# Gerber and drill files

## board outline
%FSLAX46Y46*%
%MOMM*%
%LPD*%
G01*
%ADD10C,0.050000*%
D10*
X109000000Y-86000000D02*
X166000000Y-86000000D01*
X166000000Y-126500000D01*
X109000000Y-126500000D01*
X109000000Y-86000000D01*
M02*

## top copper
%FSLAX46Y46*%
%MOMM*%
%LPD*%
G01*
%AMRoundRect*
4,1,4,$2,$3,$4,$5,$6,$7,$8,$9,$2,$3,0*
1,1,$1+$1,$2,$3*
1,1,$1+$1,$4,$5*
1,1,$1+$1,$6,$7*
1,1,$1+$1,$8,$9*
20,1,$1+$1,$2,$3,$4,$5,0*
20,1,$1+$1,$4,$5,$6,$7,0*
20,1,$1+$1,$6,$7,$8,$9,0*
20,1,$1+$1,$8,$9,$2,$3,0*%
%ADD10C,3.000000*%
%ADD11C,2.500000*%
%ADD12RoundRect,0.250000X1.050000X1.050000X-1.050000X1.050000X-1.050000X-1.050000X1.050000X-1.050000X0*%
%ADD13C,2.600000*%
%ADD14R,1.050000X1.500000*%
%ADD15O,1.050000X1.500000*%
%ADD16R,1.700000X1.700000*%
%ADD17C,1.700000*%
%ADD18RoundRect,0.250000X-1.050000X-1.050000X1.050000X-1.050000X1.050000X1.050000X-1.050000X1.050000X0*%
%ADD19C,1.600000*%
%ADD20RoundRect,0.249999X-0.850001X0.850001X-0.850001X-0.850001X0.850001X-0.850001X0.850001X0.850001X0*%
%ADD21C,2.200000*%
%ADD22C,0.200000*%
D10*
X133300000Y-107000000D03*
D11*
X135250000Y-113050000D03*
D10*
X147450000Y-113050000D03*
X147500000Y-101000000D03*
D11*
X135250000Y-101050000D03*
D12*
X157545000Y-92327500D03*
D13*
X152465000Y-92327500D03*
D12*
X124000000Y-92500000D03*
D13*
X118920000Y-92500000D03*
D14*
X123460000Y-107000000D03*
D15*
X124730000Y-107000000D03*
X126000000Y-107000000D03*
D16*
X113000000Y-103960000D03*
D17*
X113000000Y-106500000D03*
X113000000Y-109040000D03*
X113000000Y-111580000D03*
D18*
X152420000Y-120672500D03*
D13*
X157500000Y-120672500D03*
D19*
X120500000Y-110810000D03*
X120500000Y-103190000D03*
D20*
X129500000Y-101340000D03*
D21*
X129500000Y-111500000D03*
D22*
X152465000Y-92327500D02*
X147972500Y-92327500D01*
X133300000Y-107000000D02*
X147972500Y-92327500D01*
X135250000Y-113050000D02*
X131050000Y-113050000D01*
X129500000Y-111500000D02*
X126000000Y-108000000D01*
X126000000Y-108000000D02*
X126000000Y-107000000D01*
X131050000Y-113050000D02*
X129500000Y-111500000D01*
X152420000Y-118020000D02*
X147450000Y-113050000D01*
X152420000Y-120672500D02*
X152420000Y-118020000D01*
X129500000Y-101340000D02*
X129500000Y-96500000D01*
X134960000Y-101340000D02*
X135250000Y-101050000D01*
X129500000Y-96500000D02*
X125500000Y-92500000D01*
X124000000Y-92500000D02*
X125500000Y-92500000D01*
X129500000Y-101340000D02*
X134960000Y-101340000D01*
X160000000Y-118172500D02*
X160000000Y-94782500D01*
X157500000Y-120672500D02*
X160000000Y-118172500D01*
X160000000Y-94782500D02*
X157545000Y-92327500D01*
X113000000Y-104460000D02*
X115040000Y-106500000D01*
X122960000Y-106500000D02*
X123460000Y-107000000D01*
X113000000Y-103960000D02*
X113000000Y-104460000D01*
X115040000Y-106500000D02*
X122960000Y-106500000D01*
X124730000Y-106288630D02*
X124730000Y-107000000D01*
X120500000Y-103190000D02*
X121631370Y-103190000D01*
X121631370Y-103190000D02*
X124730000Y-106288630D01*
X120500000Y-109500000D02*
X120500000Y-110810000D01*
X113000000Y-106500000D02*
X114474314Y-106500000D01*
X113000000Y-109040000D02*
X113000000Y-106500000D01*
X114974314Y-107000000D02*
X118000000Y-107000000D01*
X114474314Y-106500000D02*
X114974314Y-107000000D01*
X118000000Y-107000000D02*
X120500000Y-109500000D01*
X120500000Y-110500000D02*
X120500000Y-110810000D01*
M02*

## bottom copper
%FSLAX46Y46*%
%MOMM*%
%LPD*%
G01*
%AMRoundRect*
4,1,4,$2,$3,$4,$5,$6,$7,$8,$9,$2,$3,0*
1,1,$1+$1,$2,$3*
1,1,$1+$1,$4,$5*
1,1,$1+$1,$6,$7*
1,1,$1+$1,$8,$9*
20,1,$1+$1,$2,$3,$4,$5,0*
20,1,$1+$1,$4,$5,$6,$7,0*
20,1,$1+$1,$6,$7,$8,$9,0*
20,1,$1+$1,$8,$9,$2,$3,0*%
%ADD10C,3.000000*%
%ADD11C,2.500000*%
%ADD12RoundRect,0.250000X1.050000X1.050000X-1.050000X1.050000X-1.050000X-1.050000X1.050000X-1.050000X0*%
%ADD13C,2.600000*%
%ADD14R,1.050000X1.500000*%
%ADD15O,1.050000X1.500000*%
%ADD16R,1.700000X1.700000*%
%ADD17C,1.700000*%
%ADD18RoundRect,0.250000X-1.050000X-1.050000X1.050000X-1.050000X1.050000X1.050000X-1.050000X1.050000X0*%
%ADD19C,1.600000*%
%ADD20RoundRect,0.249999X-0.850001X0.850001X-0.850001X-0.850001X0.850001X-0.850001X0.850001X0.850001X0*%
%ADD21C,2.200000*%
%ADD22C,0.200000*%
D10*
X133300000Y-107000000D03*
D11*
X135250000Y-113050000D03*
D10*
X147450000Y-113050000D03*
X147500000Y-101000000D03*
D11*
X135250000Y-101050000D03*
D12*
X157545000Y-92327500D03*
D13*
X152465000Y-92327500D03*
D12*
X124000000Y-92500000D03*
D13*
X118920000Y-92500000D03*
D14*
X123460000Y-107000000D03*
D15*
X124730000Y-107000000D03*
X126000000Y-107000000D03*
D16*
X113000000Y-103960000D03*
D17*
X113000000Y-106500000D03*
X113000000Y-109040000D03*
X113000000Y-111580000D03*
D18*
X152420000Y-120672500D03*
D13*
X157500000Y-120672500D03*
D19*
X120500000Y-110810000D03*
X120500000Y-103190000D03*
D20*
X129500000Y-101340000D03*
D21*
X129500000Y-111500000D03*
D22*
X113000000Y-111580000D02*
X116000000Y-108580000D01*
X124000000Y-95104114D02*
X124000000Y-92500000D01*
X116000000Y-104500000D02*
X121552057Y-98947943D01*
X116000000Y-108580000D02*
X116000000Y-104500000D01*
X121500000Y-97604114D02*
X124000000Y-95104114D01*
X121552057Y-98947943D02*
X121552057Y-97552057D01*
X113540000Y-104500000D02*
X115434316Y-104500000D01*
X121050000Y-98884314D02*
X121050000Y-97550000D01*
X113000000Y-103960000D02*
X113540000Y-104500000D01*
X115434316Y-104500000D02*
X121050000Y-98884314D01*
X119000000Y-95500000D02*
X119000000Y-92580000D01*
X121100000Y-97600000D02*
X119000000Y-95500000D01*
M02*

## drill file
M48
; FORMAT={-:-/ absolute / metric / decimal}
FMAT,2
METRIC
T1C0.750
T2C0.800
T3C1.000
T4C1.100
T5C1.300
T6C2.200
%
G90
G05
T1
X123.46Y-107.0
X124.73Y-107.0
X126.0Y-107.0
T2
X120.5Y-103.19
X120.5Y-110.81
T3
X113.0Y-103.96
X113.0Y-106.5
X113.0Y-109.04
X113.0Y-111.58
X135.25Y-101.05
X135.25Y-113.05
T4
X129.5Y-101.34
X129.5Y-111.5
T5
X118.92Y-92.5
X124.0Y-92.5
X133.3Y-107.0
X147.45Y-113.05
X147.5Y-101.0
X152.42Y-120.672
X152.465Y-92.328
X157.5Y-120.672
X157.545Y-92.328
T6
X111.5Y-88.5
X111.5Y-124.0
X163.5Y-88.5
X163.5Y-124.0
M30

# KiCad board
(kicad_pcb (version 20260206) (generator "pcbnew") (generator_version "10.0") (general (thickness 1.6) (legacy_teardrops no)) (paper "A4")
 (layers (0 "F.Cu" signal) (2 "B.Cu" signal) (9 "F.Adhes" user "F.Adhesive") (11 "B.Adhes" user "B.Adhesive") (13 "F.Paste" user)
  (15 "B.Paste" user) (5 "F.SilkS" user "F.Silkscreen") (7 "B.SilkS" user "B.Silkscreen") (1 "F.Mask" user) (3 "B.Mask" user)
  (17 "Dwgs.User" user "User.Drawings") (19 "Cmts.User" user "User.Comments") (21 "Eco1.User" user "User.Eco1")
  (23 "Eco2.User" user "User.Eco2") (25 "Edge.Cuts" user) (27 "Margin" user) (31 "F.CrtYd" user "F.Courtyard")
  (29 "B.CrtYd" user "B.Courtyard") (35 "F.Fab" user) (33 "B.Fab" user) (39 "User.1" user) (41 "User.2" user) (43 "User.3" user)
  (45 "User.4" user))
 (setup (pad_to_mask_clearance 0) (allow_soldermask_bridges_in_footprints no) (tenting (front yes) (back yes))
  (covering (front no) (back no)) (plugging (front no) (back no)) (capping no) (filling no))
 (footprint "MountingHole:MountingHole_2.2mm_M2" (layer "F.Cu") (at 163.5 124)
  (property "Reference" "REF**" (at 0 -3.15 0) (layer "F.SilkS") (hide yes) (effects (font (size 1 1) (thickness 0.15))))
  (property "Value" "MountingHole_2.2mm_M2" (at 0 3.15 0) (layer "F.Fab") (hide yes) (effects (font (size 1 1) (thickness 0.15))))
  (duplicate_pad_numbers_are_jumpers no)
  (pad "" np_thru_hole circle (at 0 0) (size 2.2 2.2) (drill 2.2) (layers "*.Cu" "*.Mask")))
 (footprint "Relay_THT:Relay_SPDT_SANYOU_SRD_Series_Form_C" (layer "F.Cu") (at 133.3 107)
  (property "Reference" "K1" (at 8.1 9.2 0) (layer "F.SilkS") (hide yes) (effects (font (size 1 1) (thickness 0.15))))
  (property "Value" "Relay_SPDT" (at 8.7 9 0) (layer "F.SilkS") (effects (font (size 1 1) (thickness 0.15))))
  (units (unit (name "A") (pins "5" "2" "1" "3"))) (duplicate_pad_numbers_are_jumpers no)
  (pad "1" thru_hole circle (at 0 0 90) (size 3 3) (drill 1.3) (layers "*.Cu" "*.Mask") (remove_unused_layers no) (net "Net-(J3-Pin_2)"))
  (pad "2" thru_hole circle (at 1.95 6.05 90) (size 2.5 2.5) (drill 1) (layers "*.Cu" "*.Mask") (remove_unused_layers no) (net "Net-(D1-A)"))
  (pad "3" thru_hole circle (at 14.15 6.05 90) (size 3 3) (drill 1.3) (layers "*.Cu" "*.Mask") (remove_unused_layers no)
   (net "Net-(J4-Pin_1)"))
  (pad "4" thru_hole circle (at 14.2 -6 90) (size 3 3) (drill 1.3) (layers "*.Cu" "*.Mask") (remove_unused_layers no))
  (pad "5" thru_hole circle (at 1.95 -5.95 90) (size 2.5 2.5) (drill 1) (layers "*.Cu" "*.Mask") (remove_unused_layers no) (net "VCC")))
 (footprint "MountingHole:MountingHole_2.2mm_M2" (layer "F.Cu") (at 111.5 124)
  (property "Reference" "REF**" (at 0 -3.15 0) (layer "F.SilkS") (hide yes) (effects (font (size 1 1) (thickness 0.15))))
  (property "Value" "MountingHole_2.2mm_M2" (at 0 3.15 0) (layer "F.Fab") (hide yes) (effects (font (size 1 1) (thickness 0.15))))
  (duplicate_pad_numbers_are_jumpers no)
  (pad "" np_thru_hole circle (at 0 0) (size 2.2 2.2) (drill 2.2) (layers "*.Cu" "*.Mask")))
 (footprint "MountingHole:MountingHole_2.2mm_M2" (layer "F.Cu") (at 163.5 88.5)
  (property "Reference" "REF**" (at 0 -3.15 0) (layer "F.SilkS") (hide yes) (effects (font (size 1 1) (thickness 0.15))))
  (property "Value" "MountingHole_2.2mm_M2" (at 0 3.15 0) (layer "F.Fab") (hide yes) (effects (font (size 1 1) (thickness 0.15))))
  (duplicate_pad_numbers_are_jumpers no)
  (pad "" np_thru_hole circle (at 0 0) (size 2.2 2.2) (drill 2.2) (layers "*.Cu" "*.Mask")))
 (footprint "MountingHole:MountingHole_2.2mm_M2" (layer "F.Cu") (at 111.5 88.5)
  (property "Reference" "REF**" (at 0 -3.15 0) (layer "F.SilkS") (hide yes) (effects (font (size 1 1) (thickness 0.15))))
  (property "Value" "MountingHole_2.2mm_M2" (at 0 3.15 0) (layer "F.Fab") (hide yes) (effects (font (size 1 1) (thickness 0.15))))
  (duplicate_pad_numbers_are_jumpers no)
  (pad "" np_thru_hole circle (at 0 0) (size 2.2 2.2) (drill 2.2) (layers "*.Cu" "*.Mask")))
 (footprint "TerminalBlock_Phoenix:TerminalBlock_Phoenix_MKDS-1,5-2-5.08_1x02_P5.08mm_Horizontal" (layer "F.Cu") (at 157.545 92.3275 180)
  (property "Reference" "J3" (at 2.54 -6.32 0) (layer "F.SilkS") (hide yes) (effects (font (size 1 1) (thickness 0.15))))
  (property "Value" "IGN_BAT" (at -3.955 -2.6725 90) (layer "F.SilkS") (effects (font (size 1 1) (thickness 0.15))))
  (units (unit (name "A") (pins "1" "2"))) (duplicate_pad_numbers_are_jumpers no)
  (pad "1" thru_hole roundrect (at 0 0 180) (size 2.6 2.6) (drill 1.3) (layers "*.Cu" "*.Mask") (remove_unused_layers no)
   (roundrect_rratio 0.096154) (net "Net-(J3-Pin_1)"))
  (pad "2" thru_hole circle (at 5.08 0 180) (size 2.6 2.6) (drill 1.3) (layers "*.Cu" "*.Mask") (remove_unused_layers no)
   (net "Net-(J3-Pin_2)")))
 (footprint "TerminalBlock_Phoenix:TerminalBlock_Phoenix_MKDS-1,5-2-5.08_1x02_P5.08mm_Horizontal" (layer "F.Cu") (at 124 92.5 180)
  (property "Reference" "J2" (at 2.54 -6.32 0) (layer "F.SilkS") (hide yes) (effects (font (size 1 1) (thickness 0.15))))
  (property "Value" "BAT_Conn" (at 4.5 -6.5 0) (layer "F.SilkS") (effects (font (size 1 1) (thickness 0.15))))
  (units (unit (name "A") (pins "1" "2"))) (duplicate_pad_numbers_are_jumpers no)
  (pad "1" thru_hole roundrect (at 0 0 180) (size 2.6 2.6) (drill 1.3) (layers "*.Cu" "*.Mask") (remove_unused_layers no)
   (roundrect_rratio 0.096154) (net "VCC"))
  (pad "2" thru_hole circle (at 5.08 0 180) (size 2.6 2.6) (drill 1.3) (layers "*.Cu" "*.Mask") (remove_unused_layers no) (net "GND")))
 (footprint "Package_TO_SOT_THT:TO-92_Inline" (layer "F.Cu") (at 123.46 107)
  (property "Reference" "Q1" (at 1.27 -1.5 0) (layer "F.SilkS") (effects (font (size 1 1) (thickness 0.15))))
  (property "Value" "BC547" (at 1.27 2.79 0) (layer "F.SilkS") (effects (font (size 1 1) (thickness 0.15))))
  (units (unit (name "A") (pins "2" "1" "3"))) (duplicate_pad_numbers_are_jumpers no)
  (pad "1" thru_hole rect (at 0 0) (size 1.05 1.5) (drill 0.75) (layers "*.Cu" "*.Mask") (remove_unused_layers no) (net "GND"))
  (pad "2" thru_hole oval (at 1.27 0) (size 1.05 1.5) (drill 0.75) (layers "*.Cu" "*.Mask") (remove_unused_layers no) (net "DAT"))
  (pad "3" thru_hole oval (at 2.54 0) (size 1.05 1.5) (drill 0.75) (layers "*.Cu" "*.Mask") (remove_unused_layers no) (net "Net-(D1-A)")))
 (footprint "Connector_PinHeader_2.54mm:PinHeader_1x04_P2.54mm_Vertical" (layer "F.Cu") (at 113 103.96)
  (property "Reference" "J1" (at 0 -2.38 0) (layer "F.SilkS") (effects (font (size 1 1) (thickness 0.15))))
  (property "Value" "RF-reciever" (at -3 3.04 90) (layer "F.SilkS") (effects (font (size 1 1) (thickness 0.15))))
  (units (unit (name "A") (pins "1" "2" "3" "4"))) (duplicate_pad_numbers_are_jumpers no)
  (pad "1" thru_hole rect (at 0 0) (size 1.7 1.7) (drill 1) (layers "*.Cu" "*.Mask") (remove_unused_layers no) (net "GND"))
  (pad "2" thru_hole circle (at 0 2.54) (size 1.7 1.7) (drill 1) (layers "*.Cu" "*.Mask") (remove_unused_layers no) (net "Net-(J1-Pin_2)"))
  (pad "3" thru_hole circle (at 0 5.08) (size 1.7 1.7) (drill 1) (layers "*.Cu" "*.Mask") (remove_unused_layers no) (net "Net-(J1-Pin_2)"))
  (pad "4" thru_hole circle (at 0 7.62) (size 1.7 1.7) (drill 1) (layers "*.Cu" "*.Mask") (remove_unused_layers no) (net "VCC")))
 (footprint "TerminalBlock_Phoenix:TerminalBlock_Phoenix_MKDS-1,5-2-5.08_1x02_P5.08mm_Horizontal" (layer "F.Cu") (at 152.42 120.6725)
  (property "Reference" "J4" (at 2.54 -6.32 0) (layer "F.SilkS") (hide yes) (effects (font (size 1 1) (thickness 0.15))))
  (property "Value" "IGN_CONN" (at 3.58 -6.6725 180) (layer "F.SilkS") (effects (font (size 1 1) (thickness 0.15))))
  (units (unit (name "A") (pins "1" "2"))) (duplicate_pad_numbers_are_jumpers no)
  (pad "1" thru_hole roundrect (at 0 0) (size 2.6 2.6) (drill 1.3) (layers "*.Cu" "*.Mask") (remove_unused_layers no)
   (roundrect_rratio 0.096154) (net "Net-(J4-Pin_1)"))
  (pad "2" thru_hole circle (at 5.08 0) (size 2.6 2.6) (drill 1.3) (layers "*.Cu" "*.Mask") (remove_unused_layers no) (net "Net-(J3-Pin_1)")))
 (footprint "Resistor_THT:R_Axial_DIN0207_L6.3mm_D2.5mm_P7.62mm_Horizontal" (layer "F.Cu") (at 120.5 110.81 90)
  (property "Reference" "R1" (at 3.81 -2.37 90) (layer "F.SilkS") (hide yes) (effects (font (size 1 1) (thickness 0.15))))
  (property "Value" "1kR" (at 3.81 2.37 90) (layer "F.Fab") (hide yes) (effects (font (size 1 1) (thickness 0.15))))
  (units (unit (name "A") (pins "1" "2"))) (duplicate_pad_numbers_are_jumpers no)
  (pad "1" thru_hole circle (at 0 0 90) (size 1.6 1.6) (drill 0.8) (layers "*.Cu" "*.Mask") (remove_unused_layers no) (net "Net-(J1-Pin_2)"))
  (pad "2" thru_hole circle (at 7.62 0 90) (size 1.6 1.6) (drill 0.8) (layers "*.Cu" "*.Mask") (remove_unused_layers no) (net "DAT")))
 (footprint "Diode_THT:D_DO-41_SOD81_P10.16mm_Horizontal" (layer "F.Cu") (at 129.5 101.34 -90)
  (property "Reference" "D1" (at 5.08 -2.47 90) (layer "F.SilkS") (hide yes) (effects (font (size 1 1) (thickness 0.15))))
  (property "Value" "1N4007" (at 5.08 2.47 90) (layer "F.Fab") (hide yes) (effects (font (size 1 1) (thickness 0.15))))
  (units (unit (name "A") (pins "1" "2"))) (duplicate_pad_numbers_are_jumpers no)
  (pad "1" thru_hole roundrect (at 0 0 270) (size 2.2 2.2) (drill 1.1) (layers "*.Cu" "*.Mask") (remove_unused_layers no)
   (roundrect_rratio 0.113636) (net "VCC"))
  (pad "2" thru_hole circle (at 10.16 0 270) (size 2.2 2.2) (drill 1.1) (layers "*.Cu" "*.Mask") (remove_unused_layers no)
   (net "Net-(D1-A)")))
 (gr_rect (start 109 86) (end 166 126.5) (stroke (width 0.05) (type default)) (fill no) (layer "Edge.Cuts"))
 (segment (start 152.465 92.3275) (end 147.9725 92.3275) (width 0.2) (layer "F.Cu") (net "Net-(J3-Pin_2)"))
 (segment (start 133.3 107) (end 147.9725 92.3275) (width 0.2) (layer "F.Cu") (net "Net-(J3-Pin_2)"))
 (segment (start 135.25 113.05) (end 131.05 113.05) (width 0.2) (layer "F.Cu") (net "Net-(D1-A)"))
 (segment (start 129.5 111.5) (end 126 108) (width 0.2) (layer "F.Cu") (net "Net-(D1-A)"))
 (segment (start 126 108) (end 126 107) (width 0.2) (layer "F.Cu") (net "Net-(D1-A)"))
 (segment (start 131.05 113.05) (end 129.5 111.5) (width 0.2) (layer "F.Cu") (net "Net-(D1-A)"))
 (segment (start 152.42 118.02) (end 147.45 113.05) (width 0.2) (layer "F.Cu") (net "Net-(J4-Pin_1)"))
 (segment (start 152.42 120.6725) (end 152.42 118.02) (width 0.2) (layer "F.Cu") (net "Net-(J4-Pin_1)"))
 (segment (start 129.5 101.34) (end 129.5 96.5) (width 0.2) (layer "F.Cu") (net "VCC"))
 (segment (start 134.96 101.34) (end 135.25 101.05) (width 0.2) (layer "F.Cu") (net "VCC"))
 (segment (start 129.5 96.5) (end 125.5 92.5) (width 0.2) (layer "F.Cu") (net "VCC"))
 (segment (start 124 92.5) (end 125.5 92.5) (width 0.2) (layer "F.Cu") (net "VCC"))
 (segment (start 129.5 101.34) (end 134.96 101.34) (width 0.2) (layer "F.Cu") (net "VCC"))
 (segment (start 113 111.58) (end 116 108.58) (width 0.2) (layer "B.Cu") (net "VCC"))
 (segment (start 124 95.104114) (end 124 92.5) (width 0.2) (layer "B.Cu") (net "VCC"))
 (segment (start 116 104.5) (end 121.552057 98.947943) (width 0.2) (layer "B.Cu") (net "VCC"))
 (segment (start 116 108.58) (end 116 104.5) (width 0.2) (layer "B.Cu") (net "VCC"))
 (segment (start 121.5 97.604114) (end 124 95.104114) (width 0.2) (layer "B.Cu") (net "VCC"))
 (segment (start 121.552057 98.947943) (end 121.552057 97.552057) (width 0.2) (layer "B.Cu") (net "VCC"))
 (segment (start 160 118.1725) (end 160 94.7825) (width 0.2) (layer "F.Cu") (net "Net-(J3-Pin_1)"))
 (segment (start 157.5 120.6725) (end 160 118.1725) (width 0.2) (layer "F.Cu") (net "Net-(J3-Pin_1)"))
 (segment (start 160 94.7825) (end 157.545 92.3275) (width 0.2) (layer "F.Cu") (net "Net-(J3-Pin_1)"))
 (segment (start 113 104.46) (end 115.04 106.5) (width 0.2) (layer "F.Cu") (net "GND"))
 (segment (start 122.96 106.5) (end 123.46 107) (width 0.2) (layer "F.Cu") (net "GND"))
 (segment (start 113 103.96) (end 113 104.46) (width 0.2) (layer "F.Cu") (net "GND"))
 (segment (start 115.04 106.5) (end 122.96 106.5) (width 0.2) (layer "F.Cu") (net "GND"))
 (segment (start 113.54 104.5) (end 115.434316 104.5) (width 0.2) (layer "B.Cu") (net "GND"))
 (segment (start 121.05 98.884314) (end 121.05 97.55) (width 0.2) (layer "B.Cu") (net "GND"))
 (segment (start 113 103.96) (end 113.54 104.5) (width 0.2) (layer "B.Cu") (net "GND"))
 (segment (start 115.434316 104.5) (end 121.05 98.884314) (width 0.2) (layer "B.Cu") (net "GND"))
 (segment (start 119 95.5) (end 119 92.58) (width 0.2) (layer "B.Cu") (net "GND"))
 (segment (start 121.1 97.6) (end 119 95.5) (width 0.2) (layer "B.Cu") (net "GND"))
 (segment (start 124.73 106.28863) (end 124.73 107) (width 0.2) (layer "F.Cu") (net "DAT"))
 (segment (start 120.5 103.19) (end 121.63137 103.19) (width 0.2) (layer "F.Cu") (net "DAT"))
 (segment (start 121.63137 103.19) (end 124.73 106.28863) (width 0.2) (layer "F.Cu") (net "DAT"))
 (segment (start 120.5 109.5) (end 120.5 110.81) (width 0.2) (layer "F.Cu") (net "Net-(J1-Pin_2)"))
 (segment (start 113 106.5) (end 114.474314 106.5) (width 0.2) (layer "F.Cu") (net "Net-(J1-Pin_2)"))
 (segment (start 113 109.04) (end 113 106.5) (width 0.2) (layer "F.Cu") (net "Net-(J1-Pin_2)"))
 (segment (start 114.974314 107) (end 118 107) (width 0.2) (layer "F.Cu") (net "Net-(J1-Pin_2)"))
 (segment (start 114.474314 106.5) (end 114.974314 107) (width 0.2) (layer "F.Cu") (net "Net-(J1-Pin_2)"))
 (segment (start 118 107) (end 120.5 109.5) (width 0.2) (layer "F.Cu") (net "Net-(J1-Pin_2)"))
 (segment (start 120.5 110.5) (end 120.5 110.81) (width 0.2) (layer "F.Cu") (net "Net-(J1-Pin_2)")))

